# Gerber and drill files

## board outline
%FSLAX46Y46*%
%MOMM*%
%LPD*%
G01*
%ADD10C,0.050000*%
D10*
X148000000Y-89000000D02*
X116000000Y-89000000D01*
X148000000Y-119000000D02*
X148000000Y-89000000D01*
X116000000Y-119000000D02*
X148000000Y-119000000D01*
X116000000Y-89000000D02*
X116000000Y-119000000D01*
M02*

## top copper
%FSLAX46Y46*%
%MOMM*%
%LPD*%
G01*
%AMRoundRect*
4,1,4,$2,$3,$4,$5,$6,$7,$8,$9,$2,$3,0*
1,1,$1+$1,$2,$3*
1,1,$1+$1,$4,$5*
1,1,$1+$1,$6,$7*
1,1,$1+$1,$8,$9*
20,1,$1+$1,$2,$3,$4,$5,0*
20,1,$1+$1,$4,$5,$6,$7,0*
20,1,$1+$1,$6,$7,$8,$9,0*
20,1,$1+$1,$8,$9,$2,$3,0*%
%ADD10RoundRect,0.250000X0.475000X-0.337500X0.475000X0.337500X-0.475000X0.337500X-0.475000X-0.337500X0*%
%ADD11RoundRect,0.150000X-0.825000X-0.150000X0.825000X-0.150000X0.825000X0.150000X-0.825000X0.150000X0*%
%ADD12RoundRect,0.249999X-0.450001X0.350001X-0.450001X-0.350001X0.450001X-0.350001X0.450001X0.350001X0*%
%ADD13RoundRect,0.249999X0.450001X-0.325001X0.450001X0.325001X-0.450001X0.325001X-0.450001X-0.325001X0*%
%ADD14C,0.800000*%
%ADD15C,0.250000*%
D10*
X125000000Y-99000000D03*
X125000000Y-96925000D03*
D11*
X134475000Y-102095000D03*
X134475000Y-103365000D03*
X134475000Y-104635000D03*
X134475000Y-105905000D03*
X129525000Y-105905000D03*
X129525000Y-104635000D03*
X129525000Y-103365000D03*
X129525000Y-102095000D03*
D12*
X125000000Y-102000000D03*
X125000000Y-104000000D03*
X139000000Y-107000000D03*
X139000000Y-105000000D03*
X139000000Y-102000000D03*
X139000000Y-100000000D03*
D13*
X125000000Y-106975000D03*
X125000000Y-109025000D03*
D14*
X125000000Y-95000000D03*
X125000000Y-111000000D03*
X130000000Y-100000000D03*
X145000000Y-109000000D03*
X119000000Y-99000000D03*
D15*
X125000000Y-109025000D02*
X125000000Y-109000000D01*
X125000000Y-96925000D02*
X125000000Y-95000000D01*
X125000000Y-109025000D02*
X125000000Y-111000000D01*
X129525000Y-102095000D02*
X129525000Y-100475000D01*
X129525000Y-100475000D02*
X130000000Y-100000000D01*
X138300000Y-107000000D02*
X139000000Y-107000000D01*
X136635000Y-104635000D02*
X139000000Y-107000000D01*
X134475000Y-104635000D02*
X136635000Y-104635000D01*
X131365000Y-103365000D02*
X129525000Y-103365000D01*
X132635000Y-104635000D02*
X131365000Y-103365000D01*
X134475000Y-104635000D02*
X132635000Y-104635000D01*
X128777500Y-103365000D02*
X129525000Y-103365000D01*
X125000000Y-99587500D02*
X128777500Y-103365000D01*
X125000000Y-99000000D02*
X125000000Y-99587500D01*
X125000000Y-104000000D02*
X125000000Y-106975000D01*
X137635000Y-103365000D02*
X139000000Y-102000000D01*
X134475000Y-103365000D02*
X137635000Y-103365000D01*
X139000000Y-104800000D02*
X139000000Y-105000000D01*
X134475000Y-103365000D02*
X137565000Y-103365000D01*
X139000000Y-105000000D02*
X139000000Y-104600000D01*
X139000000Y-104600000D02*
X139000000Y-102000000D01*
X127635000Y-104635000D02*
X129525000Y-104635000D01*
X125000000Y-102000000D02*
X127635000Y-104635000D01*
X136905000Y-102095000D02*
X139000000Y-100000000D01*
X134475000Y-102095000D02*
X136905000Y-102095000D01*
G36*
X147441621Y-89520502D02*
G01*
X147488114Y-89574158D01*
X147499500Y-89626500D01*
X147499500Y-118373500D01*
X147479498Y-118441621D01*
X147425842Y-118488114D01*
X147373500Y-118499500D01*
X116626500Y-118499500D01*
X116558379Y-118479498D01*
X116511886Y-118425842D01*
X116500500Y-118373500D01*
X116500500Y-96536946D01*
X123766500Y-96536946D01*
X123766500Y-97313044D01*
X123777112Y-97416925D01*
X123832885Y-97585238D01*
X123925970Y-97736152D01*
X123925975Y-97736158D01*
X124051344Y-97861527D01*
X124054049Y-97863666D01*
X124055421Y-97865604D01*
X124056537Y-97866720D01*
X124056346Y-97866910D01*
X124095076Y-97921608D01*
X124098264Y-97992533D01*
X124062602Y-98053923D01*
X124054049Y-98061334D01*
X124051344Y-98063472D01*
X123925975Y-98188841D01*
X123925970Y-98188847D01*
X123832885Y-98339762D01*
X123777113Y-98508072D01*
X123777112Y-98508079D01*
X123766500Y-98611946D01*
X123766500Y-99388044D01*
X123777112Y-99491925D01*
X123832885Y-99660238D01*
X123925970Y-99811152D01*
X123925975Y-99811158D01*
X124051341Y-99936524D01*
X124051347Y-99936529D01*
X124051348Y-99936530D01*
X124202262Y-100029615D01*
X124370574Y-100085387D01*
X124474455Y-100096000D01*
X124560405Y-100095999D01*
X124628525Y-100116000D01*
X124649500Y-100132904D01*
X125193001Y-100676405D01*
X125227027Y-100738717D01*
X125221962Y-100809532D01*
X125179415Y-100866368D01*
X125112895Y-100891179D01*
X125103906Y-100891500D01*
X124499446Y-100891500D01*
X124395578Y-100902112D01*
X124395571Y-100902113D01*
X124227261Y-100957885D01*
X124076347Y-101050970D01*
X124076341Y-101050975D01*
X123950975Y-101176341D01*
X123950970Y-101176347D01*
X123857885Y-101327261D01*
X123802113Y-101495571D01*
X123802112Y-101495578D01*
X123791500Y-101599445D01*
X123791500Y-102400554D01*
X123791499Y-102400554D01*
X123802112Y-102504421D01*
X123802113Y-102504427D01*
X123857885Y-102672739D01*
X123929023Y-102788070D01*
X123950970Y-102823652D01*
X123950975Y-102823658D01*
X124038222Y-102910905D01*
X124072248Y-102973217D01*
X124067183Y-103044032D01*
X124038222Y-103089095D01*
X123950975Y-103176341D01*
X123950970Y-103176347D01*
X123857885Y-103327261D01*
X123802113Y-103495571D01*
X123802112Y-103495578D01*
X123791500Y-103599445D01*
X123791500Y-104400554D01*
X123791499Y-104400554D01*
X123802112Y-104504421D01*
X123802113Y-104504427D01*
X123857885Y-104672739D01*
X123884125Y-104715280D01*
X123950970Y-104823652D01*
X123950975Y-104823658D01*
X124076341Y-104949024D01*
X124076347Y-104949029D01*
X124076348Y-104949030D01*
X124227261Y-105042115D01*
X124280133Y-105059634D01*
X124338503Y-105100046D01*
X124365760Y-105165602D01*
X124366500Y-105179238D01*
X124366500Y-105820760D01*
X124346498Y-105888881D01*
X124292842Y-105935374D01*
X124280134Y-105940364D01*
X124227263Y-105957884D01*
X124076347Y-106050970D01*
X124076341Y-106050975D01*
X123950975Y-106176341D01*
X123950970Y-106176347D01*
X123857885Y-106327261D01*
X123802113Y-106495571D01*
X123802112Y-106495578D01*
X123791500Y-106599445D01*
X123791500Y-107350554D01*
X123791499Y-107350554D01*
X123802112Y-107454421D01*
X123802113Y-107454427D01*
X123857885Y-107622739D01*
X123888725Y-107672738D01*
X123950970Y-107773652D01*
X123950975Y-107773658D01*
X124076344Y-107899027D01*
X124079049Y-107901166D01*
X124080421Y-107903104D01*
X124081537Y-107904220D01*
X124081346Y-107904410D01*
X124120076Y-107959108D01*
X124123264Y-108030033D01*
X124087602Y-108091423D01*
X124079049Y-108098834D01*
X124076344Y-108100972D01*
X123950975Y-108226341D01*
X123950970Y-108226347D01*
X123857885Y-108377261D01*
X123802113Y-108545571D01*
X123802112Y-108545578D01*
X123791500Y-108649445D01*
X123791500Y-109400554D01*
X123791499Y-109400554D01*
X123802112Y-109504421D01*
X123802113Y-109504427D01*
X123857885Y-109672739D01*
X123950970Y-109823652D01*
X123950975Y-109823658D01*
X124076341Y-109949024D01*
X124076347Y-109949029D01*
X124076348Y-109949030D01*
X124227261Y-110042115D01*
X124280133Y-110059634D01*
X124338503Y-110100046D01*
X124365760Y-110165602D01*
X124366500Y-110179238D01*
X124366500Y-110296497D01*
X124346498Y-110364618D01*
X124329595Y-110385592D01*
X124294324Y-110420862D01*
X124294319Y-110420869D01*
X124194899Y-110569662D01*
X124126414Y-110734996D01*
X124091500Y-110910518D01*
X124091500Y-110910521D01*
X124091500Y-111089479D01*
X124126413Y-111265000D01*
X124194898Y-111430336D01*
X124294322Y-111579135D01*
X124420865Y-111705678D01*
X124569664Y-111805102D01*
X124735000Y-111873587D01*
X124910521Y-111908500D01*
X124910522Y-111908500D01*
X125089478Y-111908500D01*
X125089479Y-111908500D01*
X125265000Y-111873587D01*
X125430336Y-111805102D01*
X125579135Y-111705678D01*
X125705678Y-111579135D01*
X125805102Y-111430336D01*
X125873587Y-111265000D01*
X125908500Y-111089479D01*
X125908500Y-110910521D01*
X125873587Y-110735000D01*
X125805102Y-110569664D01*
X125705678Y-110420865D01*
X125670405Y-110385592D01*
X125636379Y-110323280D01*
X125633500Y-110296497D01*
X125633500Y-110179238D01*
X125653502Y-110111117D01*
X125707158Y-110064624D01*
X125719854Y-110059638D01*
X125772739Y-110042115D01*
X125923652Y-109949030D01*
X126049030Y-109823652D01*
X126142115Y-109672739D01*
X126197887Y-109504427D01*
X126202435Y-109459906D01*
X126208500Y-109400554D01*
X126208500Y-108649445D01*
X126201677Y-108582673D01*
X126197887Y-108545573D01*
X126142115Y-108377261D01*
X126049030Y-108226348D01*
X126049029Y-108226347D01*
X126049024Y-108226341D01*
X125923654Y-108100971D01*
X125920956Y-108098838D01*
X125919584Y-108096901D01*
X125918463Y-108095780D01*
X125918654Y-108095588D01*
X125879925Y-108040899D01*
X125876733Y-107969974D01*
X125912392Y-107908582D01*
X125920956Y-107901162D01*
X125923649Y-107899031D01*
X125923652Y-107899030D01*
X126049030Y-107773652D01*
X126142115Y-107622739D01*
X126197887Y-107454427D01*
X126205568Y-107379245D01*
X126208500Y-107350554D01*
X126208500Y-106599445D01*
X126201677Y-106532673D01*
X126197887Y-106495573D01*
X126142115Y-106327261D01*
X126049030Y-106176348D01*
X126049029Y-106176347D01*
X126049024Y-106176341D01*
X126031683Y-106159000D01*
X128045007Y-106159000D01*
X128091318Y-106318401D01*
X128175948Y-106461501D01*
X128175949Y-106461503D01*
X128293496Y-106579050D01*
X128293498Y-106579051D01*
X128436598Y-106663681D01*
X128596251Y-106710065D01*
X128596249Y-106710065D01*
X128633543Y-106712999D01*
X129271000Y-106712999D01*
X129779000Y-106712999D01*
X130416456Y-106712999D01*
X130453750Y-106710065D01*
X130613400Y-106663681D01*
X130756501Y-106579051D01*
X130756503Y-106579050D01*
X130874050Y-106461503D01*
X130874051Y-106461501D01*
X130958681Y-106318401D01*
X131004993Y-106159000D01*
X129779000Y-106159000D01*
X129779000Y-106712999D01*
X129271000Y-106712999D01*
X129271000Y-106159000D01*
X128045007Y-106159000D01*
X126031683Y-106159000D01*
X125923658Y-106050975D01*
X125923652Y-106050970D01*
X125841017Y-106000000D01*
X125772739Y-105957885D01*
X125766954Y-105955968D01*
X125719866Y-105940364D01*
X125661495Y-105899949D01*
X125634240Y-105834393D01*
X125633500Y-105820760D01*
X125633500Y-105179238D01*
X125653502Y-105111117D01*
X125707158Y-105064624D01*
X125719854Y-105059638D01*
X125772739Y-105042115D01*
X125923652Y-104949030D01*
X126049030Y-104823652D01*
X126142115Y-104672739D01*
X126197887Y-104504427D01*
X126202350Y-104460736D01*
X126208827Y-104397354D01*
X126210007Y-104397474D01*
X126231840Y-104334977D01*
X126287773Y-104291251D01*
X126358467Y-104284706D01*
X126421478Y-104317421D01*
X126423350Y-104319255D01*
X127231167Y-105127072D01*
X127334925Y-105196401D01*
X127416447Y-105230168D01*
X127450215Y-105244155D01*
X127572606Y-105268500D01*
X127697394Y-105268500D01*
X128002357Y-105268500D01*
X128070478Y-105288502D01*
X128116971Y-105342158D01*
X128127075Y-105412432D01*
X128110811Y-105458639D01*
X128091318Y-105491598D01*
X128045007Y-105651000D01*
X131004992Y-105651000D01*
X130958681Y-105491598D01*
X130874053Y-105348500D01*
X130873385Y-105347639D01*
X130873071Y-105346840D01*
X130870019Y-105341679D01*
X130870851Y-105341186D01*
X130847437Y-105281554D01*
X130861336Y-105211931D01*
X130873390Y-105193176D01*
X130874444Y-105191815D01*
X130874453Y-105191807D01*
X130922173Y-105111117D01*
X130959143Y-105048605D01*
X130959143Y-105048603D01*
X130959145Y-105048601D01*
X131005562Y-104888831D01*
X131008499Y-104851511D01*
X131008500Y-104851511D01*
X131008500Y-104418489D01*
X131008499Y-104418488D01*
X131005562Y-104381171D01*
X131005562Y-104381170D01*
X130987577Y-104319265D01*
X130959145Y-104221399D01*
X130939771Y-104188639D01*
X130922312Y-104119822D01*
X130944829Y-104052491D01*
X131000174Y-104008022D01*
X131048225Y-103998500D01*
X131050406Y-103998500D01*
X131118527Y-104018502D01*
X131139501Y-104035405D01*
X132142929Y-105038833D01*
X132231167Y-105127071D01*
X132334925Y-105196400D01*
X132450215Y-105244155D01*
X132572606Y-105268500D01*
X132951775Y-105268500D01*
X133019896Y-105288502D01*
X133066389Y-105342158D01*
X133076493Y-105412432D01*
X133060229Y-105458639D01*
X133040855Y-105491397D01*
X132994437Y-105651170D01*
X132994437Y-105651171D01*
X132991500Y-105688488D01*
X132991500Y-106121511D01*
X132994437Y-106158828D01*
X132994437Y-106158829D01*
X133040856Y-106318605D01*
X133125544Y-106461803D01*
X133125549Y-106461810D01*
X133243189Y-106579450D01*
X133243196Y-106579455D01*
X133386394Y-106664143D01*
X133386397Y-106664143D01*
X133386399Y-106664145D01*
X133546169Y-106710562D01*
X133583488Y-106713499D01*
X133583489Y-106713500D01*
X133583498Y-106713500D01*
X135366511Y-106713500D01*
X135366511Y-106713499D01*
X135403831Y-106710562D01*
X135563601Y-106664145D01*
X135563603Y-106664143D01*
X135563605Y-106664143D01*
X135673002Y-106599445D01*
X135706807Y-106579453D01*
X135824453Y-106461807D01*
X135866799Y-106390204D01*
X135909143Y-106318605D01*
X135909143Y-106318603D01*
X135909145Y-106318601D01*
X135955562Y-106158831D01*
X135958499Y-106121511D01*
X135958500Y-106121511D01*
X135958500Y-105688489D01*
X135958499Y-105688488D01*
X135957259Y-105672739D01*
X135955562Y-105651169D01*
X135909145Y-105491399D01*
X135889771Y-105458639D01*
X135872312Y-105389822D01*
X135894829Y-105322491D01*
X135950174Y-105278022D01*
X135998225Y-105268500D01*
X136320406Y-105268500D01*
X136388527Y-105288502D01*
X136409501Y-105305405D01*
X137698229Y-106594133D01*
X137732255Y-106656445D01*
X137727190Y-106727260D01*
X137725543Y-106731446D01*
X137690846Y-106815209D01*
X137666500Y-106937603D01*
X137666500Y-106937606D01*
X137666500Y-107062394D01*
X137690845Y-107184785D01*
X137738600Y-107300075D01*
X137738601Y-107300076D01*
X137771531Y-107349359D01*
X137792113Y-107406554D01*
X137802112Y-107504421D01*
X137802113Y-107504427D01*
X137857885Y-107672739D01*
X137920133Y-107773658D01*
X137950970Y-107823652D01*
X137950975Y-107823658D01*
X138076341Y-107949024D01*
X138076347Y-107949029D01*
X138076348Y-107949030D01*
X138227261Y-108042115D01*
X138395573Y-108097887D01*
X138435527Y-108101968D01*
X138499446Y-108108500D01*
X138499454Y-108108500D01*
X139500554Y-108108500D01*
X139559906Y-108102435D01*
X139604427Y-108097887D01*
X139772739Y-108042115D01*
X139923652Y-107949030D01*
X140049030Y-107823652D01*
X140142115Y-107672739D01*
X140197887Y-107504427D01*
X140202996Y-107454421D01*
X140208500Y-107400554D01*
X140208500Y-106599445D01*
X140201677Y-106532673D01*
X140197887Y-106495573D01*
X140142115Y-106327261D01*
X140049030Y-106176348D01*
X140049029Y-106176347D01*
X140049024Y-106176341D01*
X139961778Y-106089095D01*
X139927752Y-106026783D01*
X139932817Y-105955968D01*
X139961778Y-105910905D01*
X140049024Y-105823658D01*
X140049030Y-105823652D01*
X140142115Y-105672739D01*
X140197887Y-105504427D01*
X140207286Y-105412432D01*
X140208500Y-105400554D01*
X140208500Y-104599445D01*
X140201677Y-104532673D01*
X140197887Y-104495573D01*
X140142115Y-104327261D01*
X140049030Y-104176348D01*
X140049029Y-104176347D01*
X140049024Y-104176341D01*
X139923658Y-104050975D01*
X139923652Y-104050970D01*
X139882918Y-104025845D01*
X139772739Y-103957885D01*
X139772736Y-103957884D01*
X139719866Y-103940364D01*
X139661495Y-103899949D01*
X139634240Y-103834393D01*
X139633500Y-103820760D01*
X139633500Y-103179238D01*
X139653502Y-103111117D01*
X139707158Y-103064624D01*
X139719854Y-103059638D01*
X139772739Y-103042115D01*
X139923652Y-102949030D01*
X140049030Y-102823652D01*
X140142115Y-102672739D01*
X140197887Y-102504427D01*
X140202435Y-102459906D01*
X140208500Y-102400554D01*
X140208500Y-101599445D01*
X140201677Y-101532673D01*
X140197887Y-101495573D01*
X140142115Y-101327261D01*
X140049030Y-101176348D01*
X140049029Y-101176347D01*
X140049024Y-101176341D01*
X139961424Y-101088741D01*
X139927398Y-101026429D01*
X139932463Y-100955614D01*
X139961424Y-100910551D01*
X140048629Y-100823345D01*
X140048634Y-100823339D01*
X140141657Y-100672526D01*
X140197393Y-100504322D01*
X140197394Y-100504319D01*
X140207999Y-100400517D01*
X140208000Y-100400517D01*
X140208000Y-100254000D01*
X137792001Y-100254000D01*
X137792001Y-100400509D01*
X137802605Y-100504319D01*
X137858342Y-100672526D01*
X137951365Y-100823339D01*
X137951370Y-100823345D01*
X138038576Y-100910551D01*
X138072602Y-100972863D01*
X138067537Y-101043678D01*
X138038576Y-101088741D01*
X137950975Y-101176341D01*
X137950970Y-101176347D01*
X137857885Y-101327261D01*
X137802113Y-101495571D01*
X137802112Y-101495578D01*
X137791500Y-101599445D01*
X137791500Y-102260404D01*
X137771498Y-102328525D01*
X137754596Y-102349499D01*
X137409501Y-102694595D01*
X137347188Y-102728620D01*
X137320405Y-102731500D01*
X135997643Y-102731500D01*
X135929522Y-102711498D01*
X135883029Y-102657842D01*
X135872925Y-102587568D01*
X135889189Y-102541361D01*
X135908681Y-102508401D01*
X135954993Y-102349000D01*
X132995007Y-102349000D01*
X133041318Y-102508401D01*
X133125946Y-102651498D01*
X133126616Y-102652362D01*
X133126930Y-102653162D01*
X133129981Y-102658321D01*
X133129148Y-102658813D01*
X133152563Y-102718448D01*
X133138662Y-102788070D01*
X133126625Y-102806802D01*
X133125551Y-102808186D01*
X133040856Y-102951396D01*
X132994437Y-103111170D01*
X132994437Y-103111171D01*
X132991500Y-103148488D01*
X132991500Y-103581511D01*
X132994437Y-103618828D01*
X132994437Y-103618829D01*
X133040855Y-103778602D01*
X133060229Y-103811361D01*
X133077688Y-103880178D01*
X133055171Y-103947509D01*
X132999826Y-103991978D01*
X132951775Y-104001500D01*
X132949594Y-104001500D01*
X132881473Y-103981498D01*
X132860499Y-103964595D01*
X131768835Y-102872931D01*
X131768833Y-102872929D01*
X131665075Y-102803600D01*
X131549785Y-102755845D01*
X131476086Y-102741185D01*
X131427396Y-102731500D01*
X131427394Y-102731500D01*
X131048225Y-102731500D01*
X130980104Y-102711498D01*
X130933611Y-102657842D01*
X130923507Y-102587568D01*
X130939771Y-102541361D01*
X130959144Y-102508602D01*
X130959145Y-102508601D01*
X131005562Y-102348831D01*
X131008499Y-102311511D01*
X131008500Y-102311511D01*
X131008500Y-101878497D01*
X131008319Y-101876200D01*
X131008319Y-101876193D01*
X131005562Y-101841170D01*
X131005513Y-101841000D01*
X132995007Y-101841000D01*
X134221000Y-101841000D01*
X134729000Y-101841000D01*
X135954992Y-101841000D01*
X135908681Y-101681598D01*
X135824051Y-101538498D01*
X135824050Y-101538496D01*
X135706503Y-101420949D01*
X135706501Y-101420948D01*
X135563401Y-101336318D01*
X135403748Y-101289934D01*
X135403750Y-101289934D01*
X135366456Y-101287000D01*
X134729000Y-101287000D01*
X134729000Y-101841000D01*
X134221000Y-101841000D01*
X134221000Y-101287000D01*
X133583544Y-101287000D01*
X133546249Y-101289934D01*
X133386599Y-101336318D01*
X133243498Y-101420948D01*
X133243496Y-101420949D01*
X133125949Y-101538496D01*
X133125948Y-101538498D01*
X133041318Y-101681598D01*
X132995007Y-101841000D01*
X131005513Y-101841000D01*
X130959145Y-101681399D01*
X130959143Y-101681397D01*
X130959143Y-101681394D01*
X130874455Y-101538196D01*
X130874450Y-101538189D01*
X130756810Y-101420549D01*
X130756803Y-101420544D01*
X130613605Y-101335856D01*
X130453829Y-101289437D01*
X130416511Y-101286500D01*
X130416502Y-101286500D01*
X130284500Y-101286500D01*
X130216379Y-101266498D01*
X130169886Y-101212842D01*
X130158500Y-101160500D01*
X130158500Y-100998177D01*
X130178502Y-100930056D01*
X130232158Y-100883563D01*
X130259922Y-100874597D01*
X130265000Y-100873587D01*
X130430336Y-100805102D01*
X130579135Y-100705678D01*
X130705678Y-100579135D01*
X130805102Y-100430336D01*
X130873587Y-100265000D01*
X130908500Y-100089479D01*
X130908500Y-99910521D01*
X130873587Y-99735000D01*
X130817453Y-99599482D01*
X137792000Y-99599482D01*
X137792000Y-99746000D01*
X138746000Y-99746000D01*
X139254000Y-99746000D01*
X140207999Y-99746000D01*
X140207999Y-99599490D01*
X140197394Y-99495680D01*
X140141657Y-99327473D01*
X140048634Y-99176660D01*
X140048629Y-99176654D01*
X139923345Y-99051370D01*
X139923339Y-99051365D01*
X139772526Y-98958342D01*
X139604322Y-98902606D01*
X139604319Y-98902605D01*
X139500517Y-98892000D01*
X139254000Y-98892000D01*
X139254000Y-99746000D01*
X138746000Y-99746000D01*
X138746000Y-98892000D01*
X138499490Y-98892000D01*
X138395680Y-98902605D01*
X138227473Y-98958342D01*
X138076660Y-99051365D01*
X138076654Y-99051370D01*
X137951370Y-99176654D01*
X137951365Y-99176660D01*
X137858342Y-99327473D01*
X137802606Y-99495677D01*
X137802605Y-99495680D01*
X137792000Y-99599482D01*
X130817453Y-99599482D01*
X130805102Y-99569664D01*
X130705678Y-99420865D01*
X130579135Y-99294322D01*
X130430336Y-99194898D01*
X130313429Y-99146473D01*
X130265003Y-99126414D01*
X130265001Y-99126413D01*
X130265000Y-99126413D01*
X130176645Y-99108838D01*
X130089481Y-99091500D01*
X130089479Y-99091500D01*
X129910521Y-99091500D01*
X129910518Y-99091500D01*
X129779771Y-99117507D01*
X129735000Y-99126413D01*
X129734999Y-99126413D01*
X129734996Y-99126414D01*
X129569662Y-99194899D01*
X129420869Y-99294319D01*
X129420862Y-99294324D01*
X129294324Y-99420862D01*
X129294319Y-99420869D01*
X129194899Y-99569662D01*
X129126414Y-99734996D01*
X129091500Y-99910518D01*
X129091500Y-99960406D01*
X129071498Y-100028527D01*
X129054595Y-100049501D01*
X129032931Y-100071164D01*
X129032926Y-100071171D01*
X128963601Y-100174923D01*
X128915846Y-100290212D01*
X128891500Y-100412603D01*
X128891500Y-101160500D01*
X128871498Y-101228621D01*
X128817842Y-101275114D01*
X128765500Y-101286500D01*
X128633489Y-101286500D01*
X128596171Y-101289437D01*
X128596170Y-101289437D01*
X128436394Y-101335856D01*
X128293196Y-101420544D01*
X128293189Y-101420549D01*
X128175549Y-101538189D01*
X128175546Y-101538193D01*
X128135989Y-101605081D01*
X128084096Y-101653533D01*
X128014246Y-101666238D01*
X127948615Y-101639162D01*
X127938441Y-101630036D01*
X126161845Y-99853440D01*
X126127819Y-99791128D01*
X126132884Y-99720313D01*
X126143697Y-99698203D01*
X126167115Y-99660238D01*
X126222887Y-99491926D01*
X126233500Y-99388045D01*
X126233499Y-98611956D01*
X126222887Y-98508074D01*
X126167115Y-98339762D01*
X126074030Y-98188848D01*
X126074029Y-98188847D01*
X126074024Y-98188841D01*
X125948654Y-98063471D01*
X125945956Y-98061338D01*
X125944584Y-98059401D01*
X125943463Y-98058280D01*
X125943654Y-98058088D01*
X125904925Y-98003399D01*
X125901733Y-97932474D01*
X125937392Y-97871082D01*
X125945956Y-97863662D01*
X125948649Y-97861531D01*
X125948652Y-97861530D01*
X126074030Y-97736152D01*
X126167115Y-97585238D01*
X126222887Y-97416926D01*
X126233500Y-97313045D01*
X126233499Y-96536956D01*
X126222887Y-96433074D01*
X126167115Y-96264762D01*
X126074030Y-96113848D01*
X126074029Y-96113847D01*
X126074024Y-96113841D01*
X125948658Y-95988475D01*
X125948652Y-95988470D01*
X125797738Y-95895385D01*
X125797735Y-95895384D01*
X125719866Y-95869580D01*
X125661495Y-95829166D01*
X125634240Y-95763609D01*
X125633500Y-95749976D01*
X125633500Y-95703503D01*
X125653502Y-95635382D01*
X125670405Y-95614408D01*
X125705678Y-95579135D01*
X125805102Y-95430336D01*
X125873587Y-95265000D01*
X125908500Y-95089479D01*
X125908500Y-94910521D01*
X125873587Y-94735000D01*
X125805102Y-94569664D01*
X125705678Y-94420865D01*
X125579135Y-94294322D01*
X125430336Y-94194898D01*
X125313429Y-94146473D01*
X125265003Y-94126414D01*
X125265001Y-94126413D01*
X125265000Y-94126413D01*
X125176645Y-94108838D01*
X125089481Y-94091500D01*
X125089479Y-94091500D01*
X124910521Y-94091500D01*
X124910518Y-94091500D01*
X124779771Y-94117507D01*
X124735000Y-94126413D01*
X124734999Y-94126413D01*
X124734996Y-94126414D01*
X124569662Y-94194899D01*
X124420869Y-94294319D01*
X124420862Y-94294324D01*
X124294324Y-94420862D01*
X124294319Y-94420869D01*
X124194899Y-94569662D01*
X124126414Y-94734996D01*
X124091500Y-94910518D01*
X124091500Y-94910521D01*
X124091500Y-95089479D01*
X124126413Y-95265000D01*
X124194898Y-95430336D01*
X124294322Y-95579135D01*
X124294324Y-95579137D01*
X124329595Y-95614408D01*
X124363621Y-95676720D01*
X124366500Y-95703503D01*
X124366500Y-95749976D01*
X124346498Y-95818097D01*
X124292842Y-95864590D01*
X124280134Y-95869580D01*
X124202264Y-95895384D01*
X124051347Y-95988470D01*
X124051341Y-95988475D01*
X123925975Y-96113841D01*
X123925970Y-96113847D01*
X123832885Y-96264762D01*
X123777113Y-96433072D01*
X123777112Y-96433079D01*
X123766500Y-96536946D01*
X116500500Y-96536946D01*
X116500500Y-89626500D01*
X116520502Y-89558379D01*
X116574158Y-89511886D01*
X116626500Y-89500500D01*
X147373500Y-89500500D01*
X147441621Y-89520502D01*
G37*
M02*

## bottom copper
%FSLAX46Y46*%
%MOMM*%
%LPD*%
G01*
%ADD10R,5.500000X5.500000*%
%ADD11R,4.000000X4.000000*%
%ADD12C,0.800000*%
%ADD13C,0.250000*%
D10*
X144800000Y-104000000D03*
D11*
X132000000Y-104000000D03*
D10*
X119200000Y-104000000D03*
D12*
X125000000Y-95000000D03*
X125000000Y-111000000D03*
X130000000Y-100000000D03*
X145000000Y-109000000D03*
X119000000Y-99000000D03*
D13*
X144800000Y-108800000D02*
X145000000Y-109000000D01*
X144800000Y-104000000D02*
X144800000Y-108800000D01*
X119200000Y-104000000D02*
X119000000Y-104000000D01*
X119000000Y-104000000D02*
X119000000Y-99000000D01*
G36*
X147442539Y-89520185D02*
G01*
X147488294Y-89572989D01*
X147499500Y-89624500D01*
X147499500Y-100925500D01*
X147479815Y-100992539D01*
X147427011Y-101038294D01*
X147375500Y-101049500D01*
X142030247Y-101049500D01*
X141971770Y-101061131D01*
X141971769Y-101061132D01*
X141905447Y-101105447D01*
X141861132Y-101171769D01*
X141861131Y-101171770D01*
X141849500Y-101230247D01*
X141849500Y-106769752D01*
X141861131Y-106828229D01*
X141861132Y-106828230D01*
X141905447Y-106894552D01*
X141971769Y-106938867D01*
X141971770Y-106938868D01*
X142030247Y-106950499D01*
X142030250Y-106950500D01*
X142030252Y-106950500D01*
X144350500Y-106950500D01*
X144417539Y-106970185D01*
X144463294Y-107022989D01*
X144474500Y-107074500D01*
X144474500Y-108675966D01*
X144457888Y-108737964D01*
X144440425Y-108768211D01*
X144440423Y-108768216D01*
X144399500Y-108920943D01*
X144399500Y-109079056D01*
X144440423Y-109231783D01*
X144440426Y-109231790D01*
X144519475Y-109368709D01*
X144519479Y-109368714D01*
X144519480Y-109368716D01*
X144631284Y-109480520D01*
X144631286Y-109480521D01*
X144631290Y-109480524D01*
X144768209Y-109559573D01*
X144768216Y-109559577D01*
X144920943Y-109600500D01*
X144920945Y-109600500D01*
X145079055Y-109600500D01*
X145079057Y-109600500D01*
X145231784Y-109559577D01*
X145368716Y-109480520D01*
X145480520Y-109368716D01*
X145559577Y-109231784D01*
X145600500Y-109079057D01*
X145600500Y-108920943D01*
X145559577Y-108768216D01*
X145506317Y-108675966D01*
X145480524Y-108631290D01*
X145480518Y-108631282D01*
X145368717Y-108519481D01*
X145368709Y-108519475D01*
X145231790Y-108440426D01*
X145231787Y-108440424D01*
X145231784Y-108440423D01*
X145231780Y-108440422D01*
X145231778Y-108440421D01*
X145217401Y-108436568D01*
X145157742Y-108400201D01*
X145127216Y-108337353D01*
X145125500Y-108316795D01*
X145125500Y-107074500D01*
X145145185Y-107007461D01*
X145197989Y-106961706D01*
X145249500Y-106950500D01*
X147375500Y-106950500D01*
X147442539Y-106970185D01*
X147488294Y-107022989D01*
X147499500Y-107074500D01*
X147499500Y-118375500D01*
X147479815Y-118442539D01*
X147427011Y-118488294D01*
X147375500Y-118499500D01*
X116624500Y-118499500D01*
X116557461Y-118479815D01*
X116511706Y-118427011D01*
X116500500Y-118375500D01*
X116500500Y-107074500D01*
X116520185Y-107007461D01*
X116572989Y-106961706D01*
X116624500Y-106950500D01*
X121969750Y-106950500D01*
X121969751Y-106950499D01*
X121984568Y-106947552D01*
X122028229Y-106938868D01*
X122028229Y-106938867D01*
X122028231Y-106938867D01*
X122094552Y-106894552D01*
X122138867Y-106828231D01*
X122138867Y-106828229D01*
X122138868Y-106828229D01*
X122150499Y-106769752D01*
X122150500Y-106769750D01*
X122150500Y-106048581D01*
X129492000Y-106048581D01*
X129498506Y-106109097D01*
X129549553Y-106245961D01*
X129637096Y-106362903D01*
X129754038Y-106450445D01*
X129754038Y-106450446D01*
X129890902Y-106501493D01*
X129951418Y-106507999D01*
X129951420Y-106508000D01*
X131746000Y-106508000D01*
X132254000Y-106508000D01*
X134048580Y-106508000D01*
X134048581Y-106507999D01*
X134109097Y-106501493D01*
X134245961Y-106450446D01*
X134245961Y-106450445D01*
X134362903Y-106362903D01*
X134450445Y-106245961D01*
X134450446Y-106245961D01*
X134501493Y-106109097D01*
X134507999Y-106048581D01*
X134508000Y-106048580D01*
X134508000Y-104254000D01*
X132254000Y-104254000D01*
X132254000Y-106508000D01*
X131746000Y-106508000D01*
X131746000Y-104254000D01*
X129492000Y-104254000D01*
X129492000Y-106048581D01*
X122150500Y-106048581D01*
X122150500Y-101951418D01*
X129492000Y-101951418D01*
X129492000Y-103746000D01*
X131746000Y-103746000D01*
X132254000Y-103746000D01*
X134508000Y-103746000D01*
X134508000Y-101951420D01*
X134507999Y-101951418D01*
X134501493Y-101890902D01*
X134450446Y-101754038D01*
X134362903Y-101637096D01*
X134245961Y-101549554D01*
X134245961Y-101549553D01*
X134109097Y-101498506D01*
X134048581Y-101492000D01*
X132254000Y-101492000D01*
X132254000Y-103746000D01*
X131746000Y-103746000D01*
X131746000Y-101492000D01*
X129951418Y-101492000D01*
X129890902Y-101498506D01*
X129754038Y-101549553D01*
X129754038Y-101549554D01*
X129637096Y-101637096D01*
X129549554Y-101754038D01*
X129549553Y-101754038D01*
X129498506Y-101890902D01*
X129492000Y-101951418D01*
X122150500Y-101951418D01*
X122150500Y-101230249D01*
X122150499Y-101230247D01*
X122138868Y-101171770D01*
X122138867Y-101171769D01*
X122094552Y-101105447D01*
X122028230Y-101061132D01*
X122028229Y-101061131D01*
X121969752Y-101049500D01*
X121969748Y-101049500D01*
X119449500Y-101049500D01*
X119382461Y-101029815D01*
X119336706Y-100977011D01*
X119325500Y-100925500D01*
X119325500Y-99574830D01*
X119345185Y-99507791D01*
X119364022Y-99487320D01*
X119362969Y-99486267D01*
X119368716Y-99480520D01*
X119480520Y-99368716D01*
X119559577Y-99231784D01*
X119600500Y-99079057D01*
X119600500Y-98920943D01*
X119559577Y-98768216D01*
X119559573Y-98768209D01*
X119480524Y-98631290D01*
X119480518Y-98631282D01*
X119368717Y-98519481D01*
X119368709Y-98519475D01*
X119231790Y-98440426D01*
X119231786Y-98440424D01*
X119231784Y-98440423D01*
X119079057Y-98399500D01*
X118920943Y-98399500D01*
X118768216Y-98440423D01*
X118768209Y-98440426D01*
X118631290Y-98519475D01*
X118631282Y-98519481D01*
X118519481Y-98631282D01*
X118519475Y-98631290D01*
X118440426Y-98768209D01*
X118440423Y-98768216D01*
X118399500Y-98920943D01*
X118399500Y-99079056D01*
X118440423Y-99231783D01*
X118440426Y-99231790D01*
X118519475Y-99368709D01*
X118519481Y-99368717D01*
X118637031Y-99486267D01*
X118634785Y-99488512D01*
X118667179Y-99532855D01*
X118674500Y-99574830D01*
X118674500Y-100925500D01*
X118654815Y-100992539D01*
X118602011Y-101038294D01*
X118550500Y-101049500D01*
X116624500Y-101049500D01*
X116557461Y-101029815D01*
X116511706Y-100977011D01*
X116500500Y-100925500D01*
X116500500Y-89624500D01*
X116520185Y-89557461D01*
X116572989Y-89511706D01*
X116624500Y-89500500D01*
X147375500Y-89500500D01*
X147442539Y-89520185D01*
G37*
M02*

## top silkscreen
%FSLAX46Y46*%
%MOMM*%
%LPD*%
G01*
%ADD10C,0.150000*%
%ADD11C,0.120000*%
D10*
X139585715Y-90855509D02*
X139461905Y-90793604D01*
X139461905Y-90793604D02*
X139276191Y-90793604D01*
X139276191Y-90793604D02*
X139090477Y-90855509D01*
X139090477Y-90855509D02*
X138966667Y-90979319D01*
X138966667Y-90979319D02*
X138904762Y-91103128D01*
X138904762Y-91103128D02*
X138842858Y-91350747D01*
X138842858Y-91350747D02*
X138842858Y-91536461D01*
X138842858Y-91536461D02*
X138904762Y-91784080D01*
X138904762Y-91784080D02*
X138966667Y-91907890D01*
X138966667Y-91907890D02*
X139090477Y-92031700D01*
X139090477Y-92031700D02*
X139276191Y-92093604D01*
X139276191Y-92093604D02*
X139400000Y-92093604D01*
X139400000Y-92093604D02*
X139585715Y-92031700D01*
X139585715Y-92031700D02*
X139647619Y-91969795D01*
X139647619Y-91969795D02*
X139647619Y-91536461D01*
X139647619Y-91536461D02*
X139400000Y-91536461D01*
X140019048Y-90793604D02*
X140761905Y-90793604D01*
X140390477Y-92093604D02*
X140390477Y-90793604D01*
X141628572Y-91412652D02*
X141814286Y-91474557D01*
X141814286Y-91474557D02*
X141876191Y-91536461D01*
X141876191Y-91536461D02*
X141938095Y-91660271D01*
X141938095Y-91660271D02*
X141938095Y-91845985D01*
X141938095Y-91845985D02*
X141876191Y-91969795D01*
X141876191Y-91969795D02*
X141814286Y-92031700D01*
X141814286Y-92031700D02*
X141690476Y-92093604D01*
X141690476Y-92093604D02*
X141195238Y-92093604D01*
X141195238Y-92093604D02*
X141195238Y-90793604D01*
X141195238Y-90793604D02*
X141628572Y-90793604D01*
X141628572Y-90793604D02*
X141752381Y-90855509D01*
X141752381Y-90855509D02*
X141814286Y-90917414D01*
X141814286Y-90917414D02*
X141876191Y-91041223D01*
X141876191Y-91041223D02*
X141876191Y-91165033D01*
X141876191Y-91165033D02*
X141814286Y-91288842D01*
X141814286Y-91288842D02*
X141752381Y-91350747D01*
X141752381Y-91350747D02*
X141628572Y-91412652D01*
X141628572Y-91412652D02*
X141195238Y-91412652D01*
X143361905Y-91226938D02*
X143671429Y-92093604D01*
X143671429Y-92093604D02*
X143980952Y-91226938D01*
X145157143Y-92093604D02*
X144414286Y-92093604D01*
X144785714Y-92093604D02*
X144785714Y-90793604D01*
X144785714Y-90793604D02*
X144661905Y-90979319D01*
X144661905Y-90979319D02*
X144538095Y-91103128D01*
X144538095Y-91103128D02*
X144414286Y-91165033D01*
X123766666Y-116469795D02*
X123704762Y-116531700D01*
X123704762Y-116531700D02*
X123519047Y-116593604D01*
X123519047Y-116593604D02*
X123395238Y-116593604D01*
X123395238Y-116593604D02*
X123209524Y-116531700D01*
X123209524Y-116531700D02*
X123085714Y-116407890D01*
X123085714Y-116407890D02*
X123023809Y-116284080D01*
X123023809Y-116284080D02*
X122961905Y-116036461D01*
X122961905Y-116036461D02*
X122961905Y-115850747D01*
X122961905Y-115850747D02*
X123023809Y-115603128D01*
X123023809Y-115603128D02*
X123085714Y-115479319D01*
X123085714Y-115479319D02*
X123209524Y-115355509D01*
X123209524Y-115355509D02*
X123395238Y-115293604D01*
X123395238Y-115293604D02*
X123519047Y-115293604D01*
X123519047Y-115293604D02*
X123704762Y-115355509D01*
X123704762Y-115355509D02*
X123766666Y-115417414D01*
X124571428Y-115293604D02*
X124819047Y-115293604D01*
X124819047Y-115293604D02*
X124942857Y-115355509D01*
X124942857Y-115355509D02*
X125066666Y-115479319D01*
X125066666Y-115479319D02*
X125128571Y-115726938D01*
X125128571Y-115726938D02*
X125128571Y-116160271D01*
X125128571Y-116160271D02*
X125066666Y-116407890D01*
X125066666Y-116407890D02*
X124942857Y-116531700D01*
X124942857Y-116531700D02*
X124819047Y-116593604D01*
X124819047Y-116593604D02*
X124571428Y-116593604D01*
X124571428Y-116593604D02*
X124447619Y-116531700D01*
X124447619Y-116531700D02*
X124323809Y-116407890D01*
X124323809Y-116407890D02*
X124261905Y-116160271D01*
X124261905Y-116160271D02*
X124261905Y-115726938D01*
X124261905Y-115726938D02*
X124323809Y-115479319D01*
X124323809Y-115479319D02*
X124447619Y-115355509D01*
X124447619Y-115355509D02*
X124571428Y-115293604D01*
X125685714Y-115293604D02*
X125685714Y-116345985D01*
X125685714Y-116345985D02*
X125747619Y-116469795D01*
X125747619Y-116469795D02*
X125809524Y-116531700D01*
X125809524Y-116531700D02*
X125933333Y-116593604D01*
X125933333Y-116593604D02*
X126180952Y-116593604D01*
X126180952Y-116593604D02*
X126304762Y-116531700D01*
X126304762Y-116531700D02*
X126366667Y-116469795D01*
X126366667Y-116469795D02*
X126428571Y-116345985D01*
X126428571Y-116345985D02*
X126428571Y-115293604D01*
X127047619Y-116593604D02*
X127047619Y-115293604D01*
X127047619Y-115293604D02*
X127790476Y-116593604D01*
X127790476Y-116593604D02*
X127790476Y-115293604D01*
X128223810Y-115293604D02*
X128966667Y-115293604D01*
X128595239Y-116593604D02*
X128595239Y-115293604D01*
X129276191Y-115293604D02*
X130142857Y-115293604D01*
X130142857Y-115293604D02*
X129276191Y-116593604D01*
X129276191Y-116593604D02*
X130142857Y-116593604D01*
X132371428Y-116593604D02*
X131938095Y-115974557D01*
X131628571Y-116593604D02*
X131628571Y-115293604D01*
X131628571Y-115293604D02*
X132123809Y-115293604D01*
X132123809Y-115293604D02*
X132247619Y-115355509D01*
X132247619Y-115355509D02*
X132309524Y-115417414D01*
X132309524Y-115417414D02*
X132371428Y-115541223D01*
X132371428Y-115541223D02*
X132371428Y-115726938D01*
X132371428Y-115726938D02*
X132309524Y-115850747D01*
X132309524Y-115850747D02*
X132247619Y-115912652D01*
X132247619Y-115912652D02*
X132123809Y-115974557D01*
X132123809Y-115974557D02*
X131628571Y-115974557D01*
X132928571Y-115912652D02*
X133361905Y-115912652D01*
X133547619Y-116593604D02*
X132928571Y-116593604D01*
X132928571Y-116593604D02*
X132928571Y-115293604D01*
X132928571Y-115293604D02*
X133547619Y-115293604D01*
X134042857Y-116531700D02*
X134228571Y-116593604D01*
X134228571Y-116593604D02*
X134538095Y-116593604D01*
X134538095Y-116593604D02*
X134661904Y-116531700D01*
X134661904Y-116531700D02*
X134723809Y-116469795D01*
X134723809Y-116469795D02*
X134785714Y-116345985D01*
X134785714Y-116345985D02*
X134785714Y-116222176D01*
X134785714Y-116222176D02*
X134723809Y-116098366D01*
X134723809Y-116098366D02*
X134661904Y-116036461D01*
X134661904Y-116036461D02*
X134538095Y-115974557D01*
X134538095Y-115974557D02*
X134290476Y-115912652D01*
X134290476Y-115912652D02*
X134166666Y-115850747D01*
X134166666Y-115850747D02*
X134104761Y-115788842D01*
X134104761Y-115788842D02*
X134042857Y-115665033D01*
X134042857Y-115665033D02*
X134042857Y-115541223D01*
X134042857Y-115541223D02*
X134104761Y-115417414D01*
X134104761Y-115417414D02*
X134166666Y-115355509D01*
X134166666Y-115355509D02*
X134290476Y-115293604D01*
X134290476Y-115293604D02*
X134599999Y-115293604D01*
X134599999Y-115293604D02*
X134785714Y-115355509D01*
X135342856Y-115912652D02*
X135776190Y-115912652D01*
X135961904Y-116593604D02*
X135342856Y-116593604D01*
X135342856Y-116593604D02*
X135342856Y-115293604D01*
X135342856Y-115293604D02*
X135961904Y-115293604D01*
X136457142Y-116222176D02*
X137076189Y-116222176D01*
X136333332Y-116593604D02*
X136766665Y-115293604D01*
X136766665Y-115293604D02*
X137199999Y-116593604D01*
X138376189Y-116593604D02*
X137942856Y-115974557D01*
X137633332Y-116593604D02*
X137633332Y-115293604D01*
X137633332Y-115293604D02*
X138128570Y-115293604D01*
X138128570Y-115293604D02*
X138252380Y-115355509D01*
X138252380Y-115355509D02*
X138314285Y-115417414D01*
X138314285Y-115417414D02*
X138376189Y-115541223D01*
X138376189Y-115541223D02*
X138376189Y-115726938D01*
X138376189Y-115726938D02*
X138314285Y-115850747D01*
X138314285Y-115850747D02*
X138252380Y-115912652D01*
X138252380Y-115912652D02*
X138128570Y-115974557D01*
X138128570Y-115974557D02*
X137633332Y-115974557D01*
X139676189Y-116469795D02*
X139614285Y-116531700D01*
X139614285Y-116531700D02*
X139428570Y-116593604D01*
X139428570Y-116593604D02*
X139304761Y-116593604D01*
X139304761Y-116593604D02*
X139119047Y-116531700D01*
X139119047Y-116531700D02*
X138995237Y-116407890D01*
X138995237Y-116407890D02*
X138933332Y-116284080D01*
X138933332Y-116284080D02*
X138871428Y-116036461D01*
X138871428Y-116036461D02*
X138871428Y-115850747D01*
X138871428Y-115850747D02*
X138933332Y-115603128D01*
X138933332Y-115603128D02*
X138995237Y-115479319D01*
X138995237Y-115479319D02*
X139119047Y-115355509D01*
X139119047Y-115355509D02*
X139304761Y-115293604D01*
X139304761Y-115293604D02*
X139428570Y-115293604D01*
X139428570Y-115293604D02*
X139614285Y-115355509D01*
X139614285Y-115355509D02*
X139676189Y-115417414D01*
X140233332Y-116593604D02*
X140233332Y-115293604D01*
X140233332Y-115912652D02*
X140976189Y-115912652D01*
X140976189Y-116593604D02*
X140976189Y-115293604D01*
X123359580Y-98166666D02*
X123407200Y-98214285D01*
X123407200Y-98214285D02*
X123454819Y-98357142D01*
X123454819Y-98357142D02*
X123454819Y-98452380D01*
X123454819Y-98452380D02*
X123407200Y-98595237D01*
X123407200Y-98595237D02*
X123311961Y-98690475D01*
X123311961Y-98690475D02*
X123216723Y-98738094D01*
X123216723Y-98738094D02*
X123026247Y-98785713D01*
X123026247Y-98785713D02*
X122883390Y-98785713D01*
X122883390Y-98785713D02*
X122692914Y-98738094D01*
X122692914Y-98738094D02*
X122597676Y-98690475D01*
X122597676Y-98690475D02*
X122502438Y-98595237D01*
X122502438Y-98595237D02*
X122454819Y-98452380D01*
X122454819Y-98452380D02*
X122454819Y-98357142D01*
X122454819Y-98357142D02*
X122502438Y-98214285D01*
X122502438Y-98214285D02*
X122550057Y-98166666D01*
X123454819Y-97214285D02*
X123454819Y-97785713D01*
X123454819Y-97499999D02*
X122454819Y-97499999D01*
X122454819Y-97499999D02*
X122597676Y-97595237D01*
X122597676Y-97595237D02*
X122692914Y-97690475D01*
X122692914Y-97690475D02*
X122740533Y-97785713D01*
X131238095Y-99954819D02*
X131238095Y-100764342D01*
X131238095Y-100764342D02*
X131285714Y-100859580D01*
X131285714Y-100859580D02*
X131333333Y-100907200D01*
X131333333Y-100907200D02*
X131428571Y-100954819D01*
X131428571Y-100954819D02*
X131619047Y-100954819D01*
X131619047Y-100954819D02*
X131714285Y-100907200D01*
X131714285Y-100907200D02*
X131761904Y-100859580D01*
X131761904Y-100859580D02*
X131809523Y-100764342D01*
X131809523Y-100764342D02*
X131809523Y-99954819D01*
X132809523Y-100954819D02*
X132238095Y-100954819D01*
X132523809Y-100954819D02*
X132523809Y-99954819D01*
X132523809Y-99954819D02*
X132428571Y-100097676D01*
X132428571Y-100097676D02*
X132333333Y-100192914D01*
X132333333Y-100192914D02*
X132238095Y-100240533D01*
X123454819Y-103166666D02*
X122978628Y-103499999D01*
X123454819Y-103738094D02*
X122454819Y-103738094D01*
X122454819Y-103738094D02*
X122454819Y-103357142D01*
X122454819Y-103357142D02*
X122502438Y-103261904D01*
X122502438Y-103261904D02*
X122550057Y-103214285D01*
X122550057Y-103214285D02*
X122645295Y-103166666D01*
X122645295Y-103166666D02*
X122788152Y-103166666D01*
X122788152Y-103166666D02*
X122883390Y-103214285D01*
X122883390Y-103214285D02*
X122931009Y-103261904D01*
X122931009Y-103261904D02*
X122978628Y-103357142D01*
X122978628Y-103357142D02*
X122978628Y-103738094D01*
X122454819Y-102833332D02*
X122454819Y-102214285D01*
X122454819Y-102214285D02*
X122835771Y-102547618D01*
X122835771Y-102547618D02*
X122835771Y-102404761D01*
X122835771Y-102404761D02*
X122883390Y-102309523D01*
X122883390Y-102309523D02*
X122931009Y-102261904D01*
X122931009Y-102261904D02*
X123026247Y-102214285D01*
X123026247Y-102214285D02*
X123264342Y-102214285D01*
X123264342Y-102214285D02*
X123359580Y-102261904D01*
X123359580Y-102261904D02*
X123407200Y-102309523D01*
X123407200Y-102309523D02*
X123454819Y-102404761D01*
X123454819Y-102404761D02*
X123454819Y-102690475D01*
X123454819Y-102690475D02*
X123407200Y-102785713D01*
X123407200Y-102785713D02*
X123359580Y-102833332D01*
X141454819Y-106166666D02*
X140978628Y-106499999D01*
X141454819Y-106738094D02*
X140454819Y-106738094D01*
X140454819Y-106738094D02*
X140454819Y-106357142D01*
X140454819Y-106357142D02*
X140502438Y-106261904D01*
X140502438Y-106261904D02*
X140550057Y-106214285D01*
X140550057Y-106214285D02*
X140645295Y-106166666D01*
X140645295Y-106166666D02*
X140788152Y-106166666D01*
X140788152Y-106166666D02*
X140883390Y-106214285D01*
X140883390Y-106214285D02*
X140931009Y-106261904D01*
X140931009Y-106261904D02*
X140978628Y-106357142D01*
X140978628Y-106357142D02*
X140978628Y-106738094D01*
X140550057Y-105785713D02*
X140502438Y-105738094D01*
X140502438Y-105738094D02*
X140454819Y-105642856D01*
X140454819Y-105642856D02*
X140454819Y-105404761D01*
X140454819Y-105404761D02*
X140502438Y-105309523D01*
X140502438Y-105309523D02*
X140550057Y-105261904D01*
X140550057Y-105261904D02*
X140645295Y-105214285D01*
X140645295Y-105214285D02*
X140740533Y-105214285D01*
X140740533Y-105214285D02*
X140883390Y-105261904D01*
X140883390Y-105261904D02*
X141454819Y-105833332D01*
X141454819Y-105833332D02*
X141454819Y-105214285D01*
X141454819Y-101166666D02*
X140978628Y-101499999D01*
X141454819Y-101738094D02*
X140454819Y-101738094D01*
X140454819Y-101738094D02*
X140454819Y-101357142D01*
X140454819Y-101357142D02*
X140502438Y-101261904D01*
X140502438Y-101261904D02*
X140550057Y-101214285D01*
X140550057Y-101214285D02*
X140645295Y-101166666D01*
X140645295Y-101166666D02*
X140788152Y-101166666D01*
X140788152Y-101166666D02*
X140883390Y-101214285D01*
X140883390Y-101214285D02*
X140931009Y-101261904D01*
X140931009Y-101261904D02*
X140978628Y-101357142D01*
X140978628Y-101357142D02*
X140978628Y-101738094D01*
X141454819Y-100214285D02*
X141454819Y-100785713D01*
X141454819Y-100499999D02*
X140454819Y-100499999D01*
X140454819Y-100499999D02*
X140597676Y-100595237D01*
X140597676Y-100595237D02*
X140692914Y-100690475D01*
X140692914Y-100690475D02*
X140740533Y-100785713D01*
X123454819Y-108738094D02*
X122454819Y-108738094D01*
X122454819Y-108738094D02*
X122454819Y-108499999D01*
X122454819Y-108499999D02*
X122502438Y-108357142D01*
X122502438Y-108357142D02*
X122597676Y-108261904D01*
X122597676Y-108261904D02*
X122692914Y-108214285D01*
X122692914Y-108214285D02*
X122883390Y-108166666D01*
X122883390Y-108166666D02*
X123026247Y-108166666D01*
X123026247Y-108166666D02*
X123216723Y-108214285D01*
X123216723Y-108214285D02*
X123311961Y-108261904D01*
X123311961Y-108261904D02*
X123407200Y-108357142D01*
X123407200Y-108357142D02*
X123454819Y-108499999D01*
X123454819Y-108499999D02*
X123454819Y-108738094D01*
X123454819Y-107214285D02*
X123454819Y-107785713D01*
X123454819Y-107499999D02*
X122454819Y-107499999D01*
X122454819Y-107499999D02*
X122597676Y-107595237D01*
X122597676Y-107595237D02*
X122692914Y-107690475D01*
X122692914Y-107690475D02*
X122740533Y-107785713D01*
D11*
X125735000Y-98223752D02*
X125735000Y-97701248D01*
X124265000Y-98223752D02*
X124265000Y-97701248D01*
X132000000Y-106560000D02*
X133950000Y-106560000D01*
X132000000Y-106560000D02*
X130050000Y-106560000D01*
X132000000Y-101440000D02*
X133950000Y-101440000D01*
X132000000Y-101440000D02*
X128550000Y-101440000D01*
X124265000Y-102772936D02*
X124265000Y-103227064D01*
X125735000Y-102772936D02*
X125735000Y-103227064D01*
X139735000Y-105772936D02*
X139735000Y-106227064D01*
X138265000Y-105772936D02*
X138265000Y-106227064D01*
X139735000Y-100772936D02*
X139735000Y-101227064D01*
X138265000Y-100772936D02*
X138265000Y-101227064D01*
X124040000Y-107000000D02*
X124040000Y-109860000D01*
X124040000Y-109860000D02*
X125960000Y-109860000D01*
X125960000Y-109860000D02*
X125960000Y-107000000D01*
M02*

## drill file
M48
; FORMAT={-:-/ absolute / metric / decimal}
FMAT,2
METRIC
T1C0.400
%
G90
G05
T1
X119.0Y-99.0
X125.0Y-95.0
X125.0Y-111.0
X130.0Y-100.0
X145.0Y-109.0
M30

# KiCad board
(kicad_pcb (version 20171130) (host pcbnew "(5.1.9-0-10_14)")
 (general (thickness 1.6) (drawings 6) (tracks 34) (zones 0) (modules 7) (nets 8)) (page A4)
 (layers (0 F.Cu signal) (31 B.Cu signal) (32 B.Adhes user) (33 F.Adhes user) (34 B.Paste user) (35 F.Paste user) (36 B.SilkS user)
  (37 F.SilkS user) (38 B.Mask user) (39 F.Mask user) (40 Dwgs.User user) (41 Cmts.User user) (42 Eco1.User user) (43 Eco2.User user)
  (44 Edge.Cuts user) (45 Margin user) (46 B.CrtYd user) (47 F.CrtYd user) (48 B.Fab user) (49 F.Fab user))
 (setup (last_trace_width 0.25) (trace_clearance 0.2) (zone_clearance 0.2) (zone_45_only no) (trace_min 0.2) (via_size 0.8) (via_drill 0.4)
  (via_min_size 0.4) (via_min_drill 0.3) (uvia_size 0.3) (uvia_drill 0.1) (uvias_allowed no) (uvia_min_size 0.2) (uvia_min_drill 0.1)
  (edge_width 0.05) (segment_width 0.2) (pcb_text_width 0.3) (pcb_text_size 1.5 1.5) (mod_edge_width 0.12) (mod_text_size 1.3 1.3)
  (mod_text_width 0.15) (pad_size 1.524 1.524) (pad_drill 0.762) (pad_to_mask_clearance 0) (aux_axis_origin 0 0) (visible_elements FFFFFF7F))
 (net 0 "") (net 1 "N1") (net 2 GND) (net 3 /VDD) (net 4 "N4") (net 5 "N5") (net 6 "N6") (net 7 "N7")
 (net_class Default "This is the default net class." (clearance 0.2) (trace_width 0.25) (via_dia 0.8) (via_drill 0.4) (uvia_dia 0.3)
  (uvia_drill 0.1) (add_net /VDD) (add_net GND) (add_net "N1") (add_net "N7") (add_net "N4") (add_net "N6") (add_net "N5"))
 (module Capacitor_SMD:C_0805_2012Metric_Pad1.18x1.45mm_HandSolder (layer F.Cu) (at 125 97.9625 90)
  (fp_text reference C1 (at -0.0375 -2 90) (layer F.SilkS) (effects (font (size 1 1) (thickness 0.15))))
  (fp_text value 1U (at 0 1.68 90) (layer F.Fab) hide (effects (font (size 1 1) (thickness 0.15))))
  (fp_line (start -0.261252 0.735) (end 0.261252 0.735) (layer F.SilkS) (width 0.12))
  (fp_line (start -0.261252 -0.735) (end 0.261252 -0.735) (layer F.SilkS) (width 0.12))
  (pad 1 smd roundrect (at -1.0375 0 90) (size 1.175 1.45) (layers F.Cu F.Paste F.Mask) (roundrect_rratio 0.2127659574468085) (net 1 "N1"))
  (pad 2 smd roundrect (at 1.0375 0 90) (size 1.175 1.45) (layers F.Cu F.Paste F.Mask) (roundrect_rratio 0.2127659574468085) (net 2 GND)))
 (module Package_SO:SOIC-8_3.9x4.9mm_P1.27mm (layer F.Cu) (at 132 104)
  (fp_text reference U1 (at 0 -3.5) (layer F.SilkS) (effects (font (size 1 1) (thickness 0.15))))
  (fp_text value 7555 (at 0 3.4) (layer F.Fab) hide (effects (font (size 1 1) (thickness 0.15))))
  (fp_line (start 0 2.56) (end 1.95 2.56) (layer F.SilkS) (width 0.12))
  (fp_line (start 0 2.56) (end -1.95 2.56) (layer F.SilkS) (width 0.12))
  (fp_line (start 0 -2.56) (end 1.95 -2.56) (layer F.SilkS) (width 0.12))
  (fp_line (start 0 -2.56) (end -3.45 -2.56) (layer F.SilkS) (width 0.12))
  (pad 8 smd roundrect (at 2.475 -1.905) (size 1.95 0.6) (layers F.Cu F.Paste F.Mask) (roundrect_rratio 0.25) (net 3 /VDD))
  (pad 7 smd roundrect (at 2.475 -0.635) (size 1.95 0.6) (layers F.Cu F.Paste F.Mask) (roundrect_rratio 0.25) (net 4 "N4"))
  (pad 6 smd roundrect (at 2.475 0.635) (size 1.95 0.6) (layers F.Cu F.Paste F.Mask) (roundrect_rratio 0.25) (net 1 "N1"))
  (pad 5 smd roundrect (at 2.475 1.905) (size 1.95 0.6) (layers F.Cu F.Paste F.Mask) (roundrect_rratio 0.25) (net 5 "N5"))
  (pad 4 smd roundrect (at -2.475 1.905) (size 1.95 0.6) (layers F.Cu F.Paste F.Mask) (roundrect_rratio 0.25) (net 3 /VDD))
  (pad 3 smd roundrect (at -2.475 0.635) (size 1.95 0.6) (layers F.Cu F.Paste F.Mask) (roundrect_rratio 0.25) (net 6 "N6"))
  (pad 2 smd roundrect (at -2.475 -0.635) (size 1.95 0.6) (layers F.Cu F.Paste F.Mask) (roundrect_rratio 0.25) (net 1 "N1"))
  (pad 1 smd roundrect (at -2.475 -1.905) (size 1.95 0.6) (layers F.Cu F.Paste F.Mask) (roundrect_rratio 0.25) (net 2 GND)))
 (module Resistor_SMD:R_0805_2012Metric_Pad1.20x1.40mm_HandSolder (layer F.Cu) (at 125 103 270)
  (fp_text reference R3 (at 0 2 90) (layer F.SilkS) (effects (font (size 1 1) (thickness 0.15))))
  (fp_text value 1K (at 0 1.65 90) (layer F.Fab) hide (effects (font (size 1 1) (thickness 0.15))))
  (fp_line (start -0.227064 0.735) (end 0.227064 0.735) (layer F.SilkS) (width 0.12))
  (fp_line (start -0.227064 -0.735) (end 0.227064 -0.735) (layer F.SilkS) (width 0.12))
  (pad 1 smd roundrect (at -1 0 270) (size 1.2 1.4) (layers F.Cu F.Paste F.Mask) (roundrect_rratio 0.2083325) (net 6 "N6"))
  (pad 2 smd roundrect (at 1 0 270) (size 1.2 1.4) (layers F.Cu F.Paste F.Mask) (roundrect_rratio 0.2083325) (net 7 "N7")))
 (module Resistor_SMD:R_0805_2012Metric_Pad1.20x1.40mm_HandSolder (layer F.Cu) (at 139 106 270)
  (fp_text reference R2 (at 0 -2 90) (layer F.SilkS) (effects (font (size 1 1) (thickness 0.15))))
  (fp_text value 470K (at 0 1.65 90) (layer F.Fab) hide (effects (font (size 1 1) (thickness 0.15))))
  (fp_line (start -0.227064 -0.735) (end 0.227064 -0.735) (layer F.SilkS) (width 0.12))
  (fp_line (start -0.227064 0.735) (end 0.227064 0.735) (layer F.SilkS) (width 0.12))
  (pad 2 smd roundrect (at 1 0 270) (size 1.2 1.4) (layers F.Cu F.Paste F.Mask) (roundrect_rratio 0.2083325) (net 1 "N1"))
  (pad 1 smd roundrect (at -1 0 270) (size 1.2 1.4) (layers F.Cu F.Paste F.Mask) (roundrect_rratio 0.2083325) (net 4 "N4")))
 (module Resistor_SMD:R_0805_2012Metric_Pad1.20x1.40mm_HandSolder (layer F.Cu) (at 139 101 270)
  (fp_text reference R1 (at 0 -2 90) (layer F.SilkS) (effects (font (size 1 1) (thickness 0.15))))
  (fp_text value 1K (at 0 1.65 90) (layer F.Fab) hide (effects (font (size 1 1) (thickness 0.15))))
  (fp_line (start -0.227064 -0.735) (end 0.227064 -0.735) (layer F.SilkS) (width 0.12))
  (fp_line (start -0.227064 0.735) (end 0.227064 0.735) (layer F.SilkS) (width 0.12))
  (pad 2 smd roundrect (at 1 0 270) (size 1.2 1.4) (layers F.Cu F.Paste F.Mask) (roundrect_rratio 0.2083325) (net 4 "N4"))
  (pad 1 smd roundrect (at -1 0 270) (size 1.2 1.4) (layers F.Cu F.Paste F.Mask) (roundrect_rratio 0.2083325) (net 3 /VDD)))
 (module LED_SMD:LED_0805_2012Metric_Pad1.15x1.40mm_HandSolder (layer F.Cu) (at 125 108 90)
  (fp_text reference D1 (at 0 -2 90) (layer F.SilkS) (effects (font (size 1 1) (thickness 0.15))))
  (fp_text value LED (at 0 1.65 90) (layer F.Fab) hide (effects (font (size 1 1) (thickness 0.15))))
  (fp_line (start 1 -0.96) (end -1.86 -0.96) (layer F.SilkS) (width 0.12))
  (fp_line (start -1.86 -0.96) (end -1.86 0.96) (layer F.SilkS) (width 0.12))
  (fp_line (start -1.86 0.96) (end 1 0.96) (layer F.SilkS) (width 0.12))
  (pad 2 smd roundrect (at 1.025 0 90) (size 1.15 1.4) (layers F.Cu F.Paste F.Mask) (roundrect_rratio 0.2173904347826087) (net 7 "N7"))
  (pad 1 smd roundrect (at -1.025 0 90) (size 1.15 1.4) (layers F.Cu F.Paste F.Mask) (roundrect_rratio 0.2173904347826087) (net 2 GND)))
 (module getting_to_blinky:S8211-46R (layer B.Cu) (at 132 104)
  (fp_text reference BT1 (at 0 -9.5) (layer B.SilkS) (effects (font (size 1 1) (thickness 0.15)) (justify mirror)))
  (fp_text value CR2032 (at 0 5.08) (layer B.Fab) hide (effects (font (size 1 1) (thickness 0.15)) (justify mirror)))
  (pad 1 smd rect (at 12.8 0) (size 5.5 5.5) (layers B.Cu B.Paste B.Mask) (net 3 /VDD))
  (pad 2 smd rect (at 0 0) (size 4 4) (layers B.Cu B.Paste B.Mask) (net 2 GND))
  (pad 1 smd rect (at -12.8 0) (size 5.5 5.5) (layers B.Cu B.Paste B.Mask) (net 3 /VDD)))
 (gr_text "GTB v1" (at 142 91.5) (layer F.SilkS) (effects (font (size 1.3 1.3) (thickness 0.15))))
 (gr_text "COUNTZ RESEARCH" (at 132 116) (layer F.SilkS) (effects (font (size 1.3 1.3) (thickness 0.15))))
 (gr_line (start 148 89) (end 116 89) (layer Edge.Cuts) (width 0.05))
 (gr_line (start 148 119) (end 148 89) (layer Edge.Cuts) (width 0.05))
 (gr_line (start 116 119) (end 148 119) (layer Edge.Cuts) (width 0.05))
 (gr_line (start 116 89) (end 116 119) (layer Edge.Cuts) (width 0.05))
 (segment (start 125 109.025) (end 125 109) (width 0.25) (layer F.Cu) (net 2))
 (segment (start 125 96.925) (end 125 95) (width 0.25) (layer F.Cu) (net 2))
 (via (at 125 95) (size 0.8) (drill 0.4) (layers F.Cu B.Cu) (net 2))
 (segment (start 125 109.025) (end 125 111) (width 0.25) (layer F.Cu) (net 2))
 (via (at 125 111) (size 0.8) (drill 0.4) (layers F.Cu B.Cu) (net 2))
 (segment (start 129.525 102.095) (end 129.525 100.475) (width 0.25) (layer F.Cu) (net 2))
 (segment (start 129.525 100.475) (end 130 100) (width 0.25) (layer F.Cu) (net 2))
 (via (at 130 100) (size 0.8) (drill 0.4) (layers F.Cu B.Cu) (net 2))
 (segment (start 138.3 107) (end 139 107) (width 0.25) (layer F.Cu) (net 1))
 (segment (start 136.635 104.635) (end 139 107) (width 0.25) (layer F.Cu) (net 1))
 (segment (start 134.475 104.635) (end 136.635 104.635) (width 0.25) (layer F.Cu) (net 1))
 (segment (start 131.365 103.365) (end 129.525 103.365) (width 0.25) (layer F.Cu) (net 1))
 (segment (start 132.635 104.635) (end 131.365 103.365) (width 0.25) (layer F.Cu) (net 1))
 (segment (start 134.475 104.635) (end 132.635 104.635) (width 0.25) (layer F.Cu) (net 1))
 (segment (start 128.7775 103.365) (end 129.525 103.365) (width 0.25) (layer F.Cu) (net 1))
 (segment (start 125 99.5875) (end 128.7775 103.365) (width 0.25) (layer F.Cu) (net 1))
 (segment (start 125 99) (end 125 99.5875) (width 0.25) (layer F.Cu) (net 1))
 (segment (start 125 104) (end 125 106.975) (width 0.25) (layer F.Cu) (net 7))
 (segment (start 137.635 103.365) (end 139 102) (width 0.25) (layer F.Cu) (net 4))
 (segment (start 134.475 103.365) (end 137.635 103.365) (width 0.25) (layer F.Cu) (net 4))
 (segment (start 139 104.8) (end 139 105) (width 0.25) (layer F.Cu) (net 4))
 (segment (start 134.475 103.365) (end 137.565 103.365) (width 0.25) (layer F.Cu) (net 4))
 (segment (start 139 105) (end 139 104.6) (width 0.25) (layer F.Cu) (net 4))
 (segment (start 139 104.6) (end 139 102) (width 0.25) (layer F.Cu) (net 4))
 (segment (start 127.635 104.635) (end 129.525 104.635) (width 0.25) (layer F.Cu) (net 6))
 (segment (start 125 102) (end 127.635 104.635) (width 0.25) (layer F.Cu) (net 6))
 (segment (start 136.905 102.095) (end 139 100) (width 0.25) (layer F.Cu) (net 3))
 (segment (start 134.475 102.095) (end 136.905 102.095) (width 0.25) (layer F.Cu) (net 3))
 (segment (start 144.8 108.8) (end 145 109) (width 0.25) (layer B.Cu) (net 3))
 (segment (start 144.8 104) (end 144.8 108.8) (width 0.25) (layer B.Cu) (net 3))
 (segment (start 119.2 104) (end 119 104) (width 0.25) (layer B.Cu) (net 3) (status 1000000))
 (via (at 145 109) (size 0.8) (drill 0.4) (layers F.Cu B.Cu) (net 3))
 (via (at 119 99) (size 0.8) (drill 0.4) (layers F.Cu B.Cu) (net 3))
 (segment (start 119 104) (end 119 99) (width 0.25) (layer B.Cu) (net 3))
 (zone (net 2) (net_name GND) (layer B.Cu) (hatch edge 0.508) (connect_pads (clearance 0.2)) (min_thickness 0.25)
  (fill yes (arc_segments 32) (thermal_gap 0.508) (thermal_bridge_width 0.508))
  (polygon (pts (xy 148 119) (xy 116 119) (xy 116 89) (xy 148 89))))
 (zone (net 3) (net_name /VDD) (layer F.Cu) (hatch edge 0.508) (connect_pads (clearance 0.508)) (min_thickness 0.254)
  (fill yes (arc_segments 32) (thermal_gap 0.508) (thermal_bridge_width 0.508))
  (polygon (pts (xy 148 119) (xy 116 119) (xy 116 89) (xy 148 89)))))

